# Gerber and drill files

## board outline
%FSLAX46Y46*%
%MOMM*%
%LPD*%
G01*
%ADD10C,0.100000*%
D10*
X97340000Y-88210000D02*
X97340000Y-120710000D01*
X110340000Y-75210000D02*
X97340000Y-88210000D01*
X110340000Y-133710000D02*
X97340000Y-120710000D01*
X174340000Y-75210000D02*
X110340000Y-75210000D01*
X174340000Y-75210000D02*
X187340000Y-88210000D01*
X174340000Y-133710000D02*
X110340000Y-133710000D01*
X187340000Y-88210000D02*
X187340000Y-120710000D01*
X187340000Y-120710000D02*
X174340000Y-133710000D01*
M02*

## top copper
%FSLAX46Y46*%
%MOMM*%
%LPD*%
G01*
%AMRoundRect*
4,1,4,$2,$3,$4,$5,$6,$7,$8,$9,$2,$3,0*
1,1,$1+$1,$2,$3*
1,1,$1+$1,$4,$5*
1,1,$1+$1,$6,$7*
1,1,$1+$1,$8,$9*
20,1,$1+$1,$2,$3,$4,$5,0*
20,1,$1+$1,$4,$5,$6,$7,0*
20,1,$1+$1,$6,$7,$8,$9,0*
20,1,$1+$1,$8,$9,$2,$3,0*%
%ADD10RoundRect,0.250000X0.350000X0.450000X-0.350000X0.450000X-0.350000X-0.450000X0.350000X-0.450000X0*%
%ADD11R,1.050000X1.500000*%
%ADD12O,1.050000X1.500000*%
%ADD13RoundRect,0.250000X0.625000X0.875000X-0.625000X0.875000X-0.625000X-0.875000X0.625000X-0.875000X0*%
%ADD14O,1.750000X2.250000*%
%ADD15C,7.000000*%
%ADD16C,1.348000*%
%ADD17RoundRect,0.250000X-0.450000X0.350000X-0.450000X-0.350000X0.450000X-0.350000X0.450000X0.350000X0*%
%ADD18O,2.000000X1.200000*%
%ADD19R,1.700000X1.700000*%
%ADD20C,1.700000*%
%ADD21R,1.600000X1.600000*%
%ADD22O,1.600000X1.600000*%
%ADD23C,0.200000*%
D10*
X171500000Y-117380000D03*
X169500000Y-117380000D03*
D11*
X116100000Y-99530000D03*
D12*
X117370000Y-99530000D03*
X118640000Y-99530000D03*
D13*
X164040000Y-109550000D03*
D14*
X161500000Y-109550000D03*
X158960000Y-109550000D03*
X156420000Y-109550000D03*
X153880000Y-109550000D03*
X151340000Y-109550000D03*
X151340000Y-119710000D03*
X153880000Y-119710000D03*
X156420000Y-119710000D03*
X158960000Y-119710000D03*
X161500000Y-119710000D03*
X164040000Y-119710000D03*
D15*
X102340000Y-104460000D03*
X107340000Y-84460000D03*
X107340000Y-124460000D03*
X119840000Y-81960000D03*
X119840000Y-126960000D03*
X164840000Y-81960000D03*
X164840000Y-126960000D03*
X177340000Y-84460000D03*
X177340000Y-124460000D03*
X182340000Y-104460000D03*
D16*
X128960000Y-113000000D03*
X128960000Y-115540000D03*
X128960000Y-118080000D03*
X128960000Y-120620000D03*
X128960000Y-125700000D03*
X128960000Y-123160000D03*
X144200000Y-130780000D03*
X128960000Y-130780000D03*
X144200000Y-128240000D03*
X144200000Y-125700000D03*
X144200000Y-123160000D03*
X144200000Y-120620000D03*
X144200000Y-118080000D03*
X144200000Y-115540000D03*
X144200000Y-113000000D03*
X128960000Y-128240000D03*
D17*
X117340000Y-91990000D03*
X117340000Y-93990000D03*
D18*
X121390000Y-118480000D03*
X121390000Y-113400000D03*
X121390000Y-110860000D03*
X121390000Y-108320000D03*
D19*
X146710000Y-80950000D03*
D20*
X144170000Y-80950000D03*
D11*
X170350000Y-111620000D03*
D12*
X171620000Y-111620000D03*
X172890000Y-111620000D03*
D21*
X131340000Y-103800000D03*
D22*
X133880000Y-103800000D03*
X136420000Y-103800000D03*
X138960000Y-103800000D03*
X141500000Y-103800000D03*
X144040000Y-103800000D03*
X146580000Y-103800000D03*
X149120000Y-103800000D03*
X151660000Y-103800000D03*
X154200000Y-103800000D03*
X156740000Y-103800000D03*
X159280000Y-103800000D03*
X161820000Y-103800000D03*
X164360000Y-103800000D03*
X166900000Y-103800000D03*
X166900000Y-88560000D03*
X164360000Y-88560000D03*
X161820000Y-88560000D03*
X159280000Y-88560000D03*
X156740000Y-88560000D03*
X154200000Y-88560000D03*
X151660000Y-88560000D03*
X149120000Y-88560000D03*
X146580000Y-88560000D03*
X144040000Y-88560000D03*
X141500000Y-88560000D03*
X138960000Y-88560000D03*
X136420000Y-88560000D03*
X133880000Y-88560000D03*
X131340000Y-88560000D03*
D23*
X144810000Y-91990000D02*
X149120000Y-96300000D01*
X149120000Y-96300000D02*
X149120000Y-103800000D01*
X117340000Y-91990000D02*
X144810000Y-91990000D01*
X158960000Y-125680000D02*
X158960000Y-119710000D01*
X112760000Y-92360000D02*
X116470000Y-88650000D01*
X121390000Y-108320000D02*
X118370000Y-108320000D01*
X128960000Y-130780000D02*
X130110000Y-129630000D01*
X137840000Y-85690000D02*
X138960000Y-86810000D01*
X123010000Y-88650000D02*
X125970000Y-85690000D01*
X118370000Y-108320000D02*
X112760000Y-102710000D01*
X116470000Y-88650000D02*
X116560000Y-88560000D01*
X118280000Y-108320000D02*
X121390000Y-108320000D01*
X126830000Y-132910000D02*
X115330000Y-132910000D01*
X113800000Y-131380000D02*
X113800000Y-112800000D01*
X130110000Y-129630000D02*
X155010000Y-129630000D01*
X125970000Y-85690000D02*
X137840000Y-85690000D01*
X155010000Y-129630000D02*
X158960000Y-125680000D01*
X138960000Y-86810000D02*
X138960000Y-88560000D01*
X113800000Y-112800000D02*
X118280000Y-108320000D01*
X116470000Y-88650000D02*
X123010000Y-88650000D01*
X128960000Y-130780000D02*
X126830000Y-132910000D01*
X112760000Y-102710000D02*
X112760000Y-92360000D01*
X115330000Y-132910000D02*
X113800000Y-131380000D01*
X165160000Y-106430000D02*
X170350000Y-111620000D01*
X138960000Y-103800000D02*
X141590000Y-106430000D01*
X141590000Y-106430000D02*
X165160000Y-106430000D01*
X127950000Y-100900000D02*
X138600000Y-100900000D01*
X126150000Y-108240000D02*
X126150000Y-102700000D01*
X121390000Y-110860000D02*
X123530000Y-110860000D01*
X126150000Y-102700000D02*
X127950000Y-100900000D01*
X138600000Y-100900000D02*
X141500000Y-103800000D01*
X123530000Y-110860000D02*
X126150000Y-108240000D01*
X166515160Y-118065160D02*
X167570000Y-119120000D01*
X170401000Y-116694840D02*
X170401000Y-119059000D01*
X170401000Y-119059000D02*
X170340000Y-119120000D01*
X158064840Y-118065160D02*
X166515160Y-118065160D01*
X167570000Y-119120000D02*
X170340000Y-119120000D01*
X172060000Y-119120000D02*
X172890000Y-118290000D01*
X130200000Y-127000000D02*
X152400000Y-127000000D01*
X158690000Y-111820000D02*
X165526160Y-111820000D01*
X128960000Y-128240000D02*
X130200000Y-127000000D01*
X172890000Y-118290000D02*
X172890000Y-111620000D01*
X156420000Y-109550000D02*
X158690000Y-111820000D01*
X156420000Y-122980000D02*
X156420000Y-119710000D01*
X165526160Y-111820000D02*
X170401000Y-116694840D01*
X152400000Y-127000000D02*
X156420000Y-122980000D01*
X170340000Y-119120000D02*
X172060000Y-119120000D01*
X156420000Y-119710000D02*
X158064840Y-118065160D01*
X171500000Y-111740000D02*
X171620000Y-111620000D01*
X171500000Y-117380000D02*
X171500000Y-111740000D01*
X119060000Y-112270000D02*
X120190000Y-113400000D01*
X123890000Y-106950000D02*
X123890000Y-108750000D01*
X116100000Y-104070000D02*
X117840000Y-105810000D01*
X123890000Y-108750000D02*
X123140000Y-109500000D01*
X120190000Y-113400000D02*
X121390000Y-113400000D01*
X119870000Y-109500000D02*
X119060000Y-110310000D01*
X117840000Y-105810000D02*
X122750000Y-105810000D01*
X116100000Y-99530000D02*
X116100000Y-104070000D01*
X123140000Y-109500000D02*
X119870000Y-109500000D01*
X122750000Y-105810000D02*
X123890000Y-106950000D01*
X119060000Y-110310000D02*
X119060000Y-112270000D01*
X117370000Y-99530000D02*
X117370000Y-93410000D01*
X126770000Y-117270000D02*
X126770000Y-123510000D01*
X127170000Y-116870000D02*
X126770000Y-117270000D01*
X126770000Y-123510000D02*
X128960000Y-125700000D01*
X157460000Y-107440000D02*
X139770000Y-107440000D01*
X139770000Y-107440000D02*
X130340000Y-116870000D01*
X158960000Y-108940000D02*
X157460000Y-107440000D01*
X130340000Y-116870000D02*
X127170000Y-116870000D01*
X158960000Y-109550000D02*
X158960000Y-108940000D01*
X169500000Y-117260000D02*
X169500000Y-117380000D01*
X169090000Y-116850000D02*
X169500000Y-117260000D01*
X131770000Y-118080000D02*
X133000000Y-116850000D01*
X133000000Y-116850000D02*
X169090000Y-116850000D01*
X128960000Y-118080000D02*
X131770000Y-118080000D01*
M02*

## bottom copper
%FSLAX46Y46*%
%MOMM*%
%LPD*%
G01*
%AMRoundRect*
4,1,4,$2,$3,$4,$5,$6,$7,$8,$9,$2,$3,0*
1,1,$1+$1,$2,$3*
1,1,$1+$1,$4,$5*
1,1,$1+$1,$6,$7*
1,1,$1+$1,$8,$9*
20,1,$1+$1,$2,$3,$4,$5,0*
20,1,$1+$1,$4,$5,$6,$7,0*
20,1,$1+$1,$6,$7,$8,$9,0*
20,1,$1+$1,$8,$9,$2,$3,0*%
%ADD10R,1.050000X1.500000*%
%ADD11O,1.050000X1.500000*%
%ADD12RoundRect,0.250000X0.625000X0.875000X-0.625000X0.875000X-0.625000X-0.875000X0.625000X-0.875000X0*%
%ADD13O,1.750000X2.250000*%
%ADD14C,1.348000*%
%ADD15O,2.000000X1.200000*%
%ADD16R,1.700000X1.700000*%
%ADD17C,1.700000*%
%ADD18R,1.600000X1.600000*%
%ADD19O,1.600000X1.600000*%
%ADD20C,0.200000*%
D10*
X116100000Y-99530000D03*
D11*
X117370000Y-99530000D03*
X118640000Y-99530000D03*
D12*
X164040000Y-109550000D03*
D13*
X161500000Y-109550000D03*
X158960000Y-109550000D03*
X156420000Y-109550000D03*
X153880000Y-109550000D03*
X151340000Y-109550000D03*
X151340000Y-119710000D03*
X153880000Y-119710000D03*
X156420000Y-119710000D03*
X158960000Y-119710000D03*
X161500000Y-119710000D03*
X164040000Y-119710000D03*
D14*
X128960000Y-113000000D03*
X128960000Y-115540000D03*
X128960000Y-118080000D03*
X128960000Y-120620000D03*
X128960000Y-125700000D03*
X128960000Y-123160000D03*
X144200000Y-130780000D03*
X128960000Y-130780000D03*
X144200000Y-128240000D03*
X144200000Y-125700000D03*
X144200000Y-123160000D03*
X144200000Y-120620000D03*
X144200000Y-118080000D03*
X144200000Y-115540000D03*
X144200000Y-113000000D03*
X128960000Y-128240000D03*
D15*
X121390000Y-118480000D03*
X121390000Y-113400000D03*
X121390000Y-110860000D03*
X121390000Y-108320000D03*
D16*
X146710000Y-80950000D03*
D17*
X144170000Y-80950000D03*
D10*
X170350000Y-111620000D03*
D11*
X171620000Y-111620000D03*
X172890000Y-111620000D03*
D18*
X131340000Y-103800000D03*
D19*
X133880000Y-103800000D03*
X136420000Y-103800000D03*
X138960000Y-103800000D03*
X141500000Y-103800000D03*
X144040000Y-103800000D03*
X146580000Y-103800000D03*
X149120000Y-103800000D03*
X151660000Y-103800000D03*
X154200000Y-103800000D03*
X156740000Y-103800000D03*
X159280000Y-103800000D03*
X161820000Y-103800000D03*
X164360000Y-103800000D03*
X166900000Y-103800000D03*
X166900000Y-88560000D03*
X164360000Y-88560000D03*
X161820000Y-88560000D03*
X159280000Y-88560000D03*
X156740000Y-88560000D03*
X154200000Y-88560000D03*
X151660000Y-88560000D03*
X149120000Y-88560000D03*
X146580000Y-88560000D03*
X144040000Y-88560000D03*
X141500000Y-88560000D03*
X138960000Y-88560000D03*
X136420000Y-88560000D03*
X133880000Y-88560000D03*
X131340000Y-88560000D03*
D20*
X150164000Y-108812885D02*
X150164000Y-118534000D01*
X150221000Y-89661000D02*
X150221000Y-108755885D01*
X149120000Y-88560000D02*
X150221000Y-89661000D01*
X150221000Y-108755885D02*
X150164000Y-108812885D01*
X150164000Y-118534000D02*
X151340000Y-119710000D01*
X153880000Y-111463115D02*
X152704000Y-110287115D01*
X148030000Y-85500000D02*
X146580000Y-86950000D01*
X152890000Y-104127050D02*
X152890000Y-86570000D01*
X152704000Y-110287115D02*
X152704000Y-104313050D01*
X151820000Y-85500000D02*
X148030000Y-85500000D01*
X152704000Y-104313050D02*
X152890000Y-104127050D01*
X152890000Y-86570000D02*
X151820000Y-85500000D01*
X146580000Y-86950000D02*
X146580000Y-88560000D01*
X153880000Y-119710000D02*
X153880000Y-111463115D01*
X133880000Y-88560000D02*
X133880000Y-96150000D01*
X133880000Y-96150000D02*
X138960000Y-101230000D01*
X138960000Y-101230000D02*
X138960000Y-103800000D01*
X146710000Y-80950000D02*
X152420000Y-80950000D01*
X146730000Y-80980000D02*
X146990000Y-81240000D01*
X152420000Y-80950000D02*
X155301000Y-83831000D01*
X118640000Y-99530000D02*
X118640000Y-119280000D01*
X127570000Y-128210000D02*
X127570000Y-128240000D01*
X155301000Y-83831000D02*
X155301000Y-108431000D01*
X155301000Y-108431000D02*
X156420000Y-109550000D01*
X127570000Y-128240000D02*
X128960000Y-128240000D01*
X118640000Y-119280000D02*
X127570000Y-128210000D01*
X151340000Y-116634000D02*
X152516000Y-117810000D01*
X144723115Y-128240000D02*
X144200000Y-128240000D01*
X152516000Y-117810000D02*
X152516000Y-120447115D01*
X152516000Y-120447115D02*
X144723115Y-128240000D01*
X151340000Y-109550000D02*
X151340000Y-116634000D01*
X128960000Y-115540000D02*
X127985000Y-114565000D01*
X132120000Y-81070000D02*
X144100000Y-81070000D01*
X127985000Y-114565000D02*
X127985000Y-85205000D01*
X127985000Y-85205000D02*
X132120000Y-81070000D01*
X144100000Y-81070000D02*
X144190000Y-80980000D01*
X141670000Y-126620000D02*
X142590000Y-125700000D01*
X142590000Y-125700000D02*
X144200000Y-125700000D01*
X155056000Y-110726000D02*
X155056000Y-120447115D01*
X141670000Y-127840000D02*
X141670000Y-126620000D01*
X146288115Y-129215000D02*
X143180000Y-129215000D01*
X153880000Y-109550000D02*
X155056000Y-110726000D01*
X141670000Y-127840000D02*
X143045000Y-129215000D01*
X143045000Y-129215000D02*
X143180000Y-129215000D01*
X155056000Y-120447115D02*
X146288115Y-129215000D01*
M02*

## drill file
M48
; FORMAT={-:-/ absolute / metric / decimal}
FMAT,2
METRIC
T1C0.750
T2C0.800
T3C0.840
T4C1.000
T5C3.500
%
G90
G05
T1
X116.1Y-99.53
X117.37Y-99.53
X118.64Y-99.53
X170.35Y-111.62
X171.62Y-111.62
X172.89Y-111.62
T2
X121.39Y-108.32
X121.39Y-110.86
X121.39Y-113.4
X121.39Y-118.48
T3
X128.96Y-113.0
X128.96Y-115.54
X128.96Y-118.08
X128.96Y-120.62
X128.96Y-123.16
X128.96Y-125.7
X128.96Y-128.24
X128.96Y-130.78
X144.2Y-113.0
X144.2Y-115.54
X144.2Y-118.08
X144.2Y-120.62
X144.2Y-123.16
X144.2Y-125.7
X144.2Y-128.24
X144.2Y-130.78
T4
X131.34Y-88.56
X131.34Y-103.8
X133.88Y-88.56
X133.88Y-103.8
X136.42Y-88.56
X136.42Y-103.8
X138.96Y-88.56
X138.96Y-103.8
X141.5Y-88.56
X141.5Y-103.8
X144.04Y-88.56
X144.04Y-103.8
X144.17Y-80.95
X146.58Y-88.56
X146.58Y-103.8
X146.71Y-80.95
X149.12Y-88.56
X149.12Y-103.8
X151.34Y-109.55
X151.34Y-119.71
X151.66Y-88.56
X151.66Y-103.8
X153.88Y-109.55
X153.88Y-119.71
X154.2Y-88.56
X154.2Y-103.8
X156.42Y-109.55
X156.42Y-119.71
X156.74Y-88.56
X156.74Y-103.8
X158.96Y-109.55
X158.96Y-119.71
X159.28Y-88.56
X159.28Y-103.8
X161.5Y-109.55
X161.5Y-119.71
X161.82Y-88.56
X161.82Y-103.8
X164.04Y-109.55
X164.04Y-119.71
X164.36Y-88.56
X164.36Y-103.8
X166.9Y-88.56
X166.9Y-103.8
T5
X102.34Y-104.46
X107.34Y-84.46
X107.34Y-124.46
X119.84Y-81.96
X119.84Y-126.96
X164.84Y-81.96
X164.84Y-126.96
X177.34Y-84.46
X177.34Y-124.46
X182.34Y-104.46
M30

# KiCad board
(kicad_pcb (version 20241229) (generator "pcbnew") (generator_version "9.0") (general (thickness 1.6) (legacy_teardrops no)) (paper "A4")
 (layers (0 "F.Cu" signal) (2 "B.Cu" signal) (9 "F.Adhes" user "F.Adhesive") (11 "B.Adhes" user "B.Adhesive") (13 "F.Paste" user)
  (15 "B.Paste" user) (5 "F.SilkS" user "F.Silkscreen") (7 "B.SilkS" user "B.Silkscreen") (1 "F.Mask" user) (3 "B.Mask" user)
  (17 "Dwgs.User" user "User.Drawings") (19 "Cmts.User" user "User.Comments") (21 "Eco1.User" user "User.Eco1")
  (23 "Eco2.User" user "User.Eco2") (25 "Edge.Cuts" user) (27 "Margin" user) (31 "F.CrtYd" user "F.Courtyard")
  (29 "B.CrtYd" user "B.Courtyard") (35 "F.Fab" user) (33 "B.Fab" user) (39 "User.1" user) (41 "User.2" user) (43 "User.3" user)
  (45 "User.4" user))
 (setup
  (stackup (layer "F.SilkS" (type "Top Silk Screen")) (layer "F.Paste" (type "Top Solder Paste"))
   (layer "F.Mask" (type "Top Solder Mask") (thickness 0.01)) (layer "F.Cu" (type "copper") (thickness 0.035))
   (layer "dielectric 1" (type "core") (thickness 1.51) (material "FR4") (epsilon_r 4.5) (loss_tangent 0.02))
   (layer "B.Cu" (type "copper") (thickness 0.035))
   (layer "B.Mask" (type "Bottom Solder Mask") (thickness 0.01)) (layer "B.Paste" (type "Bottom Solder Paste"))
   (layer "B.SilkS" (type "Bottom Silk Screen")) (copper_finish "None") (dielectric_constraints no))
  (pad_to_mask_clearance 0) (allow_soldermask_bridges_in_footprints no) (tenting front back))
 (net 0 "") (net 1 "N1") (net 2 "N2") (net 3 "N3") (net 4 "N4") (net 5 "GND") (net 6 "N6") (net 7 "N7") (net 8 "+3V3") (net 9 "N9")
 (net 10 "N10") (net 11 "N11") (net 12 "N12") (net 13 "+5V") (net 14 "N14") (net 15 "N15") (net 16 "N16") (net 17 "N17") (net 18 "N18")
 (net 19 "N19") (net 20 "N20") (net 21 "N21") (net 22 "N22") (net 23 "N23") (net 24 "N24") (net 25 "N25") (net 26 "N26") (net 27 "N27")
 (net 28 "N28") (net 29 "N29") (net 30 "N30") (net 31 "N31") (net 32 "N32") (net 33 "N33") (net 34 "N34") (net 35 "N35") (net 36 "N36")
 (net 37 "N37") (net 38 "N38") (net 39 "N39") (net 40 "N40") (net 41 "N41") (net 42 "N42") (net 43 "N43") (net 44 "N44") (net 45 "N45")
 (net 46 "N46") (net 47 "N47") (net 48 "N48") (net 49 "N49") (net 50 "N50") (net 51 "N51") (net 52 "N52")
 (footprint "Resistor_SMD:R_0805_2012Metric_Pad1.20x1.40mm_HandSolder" (layer "F.Cu") (at 170.5 117.38 180)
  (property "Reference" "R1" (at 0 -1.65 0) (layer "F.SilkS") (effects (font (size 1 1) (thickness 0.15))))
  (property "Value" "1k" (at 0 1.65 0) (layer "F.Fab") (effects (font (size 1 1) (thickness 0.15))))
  (pad "1" smd roundrect (at -1 0 180) (size 1.2 1.4) (layers "F.Cu" "F.Mask" "F.Paste") (roundrect_rratio 0.208333) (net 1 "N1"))
  (pad "2" smd roundrect (at 1 0 180) (size 1.2 1.4) (layers "F.Cu" "F.Mask" "F.Paste") (roundrect_rratio 0.208333) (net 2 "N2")))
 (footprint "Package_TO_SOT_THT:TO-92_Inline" (layer "F.Cu") (at 116.1 99.53)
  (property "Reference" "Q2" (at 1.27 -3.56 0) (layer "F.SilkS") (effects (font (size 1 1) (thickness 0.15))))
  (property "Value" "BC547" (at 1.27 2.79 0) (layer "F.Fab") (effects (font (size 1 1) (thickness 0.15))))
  (pad "1" thru_hole rect (at 0 0) (size 1.05 1.5) (drill 0.75) (layers "*.Cu" "*.Mask") (remove_unused_layers no) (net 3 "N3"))
  (pad "2" thru_hole oval (at 1.27 0) (size 1.05 1.5) (drill 0.75) (layers "*.Cu" "*.Mask") (remove_unused_layers no) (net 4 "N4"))
  (pad "3" thru_hole oval (at 2.54 0) (size 1.05 1.5) (drill 0.75) (layers "*.Cu" "*.Mask") (remove_unused_layers no) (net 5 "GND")))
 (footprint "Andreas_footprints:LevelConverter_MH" (layer "F.Cu") (at 157.69 114.63 180)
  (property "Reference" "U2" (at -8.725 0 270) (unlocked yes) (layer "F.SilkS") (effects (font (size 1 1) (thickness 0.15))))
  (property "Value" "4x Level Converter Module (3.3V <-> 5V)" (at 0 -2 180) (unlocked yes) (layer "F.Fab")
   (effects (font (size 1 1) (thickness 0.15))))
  (pad "1" thru_hole roundrect (at -6.35 5.08 180) (size 1.75 2.25) (drill 1) (layers "*.Cu" "*.Mask") (remove_unused_layers no)
   (roundrect_rratio 0.1428571429) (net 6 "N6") (thermal_bridge_angle 45))
  (pad "2" thru_hole oval (at -3.81 5.08 180) (size 1.75 2.25) (drill 1) (layers "*.Cu" "*.Mask") (remove_unused_layers no) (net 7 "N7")
   (thermal_bridge_angle 45))
  (pad "3" thru_hole oval (at -1.27 5.08 180) (size 1.75 2.25) (drill 1) (layers "*.Cu" "*.Mask") (remove_unused_layers no) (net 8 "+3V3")
   (thermal_bridge_angle 45))
  (pad "4" thru_hole oval (at 1.27 5.08 180) (size 1.75 2.25) (drill 1) (layers "*.Cu" "*.Mask") (remove_unused_layers no) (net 5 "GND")
   (thermal_bridge_angle 45))
  (pad "5" thru_hole oval (at 3.81 5.08 180) (size 1.75 2.25) (drill 1) (layers "*.Cu" "*.Mask") (remove_unused_layers no) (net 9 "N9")
   (thermal_bridge_angle 45))
  (pad "6" thru_hole oval (at 6.35 5.08 180) (size 1.75 2.25) (drill 1) (layers "*.Cu" "*.Mask") (remove_unused_layers no) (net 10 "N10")
   (thermal_bridge_angle 45))
  (pad "7" thru_hole oval (at 6.35 -5.08 180) (size 1.75 2.25) (drill 1) (layers "*.Cu" "*.Mask") (remove_unused_layers no) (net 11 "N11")
   (thermal_bridge_angle 45))
  (pad "8" thru_hole oval (at 3.81 -5.08 180) (size 1.75 2.25) (drill 1) (layers "*.Cu" "*.Mask") (remove_unused_layers no) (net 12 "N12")
   (thermal_bridge_angle 45))
  (pad "9" thru_hole oval (at 1.27 -5.08 180) (size 1.75 2.25) (drill 1) (layers "*.Cu" "*.Mask") (remove_unused_layers no) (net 5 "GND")
   (thermal_bridge_angle 45))
  (pad "10" thru_hole oval (at -1.27 -5.08 180) (size 1.75 2.25) (drill 1) (layers "*.Cu" "*.Mask") (remove_unused_layers no) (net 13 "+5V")
   (thermal_bridge_angle 45))
  (pad "11" thru_hole oval (at -3.81 -5.08 180) (size 1.75 2.25) (drill 1) (layers "*.Cu" "*.Mask") (remove_unused_layers no) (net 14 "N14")
   (thermal_bridge_angle 45))
  (pad "12" thru_hole oval (at -6.35 -5.08 180) (size 1.75 2.25) (drill 1) (layers "*.Cu" "*.Mask") (remove_unused_layers no) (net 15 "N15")
   (thermal_bridge_angle 45)))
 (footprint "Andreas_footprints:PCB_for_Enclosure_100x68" (layer "F.Cu") (at 142.34 104.46)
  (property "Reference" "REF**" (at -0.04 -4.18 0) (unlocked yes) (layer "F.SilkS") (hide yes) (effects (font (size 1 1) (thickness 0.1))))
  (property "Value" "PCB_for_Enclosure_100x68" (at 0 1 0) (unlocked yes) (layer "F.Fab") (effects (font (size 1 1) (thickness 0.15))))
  (fp_line (start -45 -16.25) (end -45 16.25) (stroke (width 0.1) (type default)) (layer "Edge.Cuts"))
  (fp_line (start -32 -29.25) (end -45 -16.25) (stroke (width 0.1) (type default)) (layer "Edge.Cuts"))
  (fp_line (start -32 29.25) (end -45 16.25) (stroke (width 0.1) (type default)) (layer "Edge.Cuts"))
  (fp_line (start 32 -29.25) (end -32 -29.25) (stroke (width 0.1) (type default)) (layer "Edge.Cuts"))
  (fp_line (start 32 -29.25) (end 45 -16.25) (stroke (width 0.1) (type default)) (layer "Edge.Cuts"))
  (fp_line (start 32 29.25) (end -32 29.25) (stroke (width 0.1) (type default)) (layer "Edge.Cuts"))
  (fp_line (start 45 -16.25) (end 45 16.25) (stroke (width 0.1) (type default)) (layer "Edge.Cuts"))
  (fp_line (start 45 16.25) (end 32 29.25) (stroke (width 0.1) (type default)) (layer "Edge.Cuts"))
  (pad "" np_thru_hole circle (at -40 0) (size 7 7) (drill 3.5) (layers "F.Cu" "F.Mask" "F.Paste"))
  (pad "" np_thru_hole circle (at -35 -20) (size 7 7) (drill 3.5) (layers "F.Cu" "F.Mask" "F.Paste"))
  (pad "" np_thru_hole circle (at -35 20) (size 7 7) (drill 3.5) (layers "F.Cu" "F.Mask" "F.Paste"))
  (pad "" np_thru_hole circle (at -22.5 -22.5) (size 7 7) (drill 3.5) (layers "F.Cu" "F.Mask" "F.Paste"))
  (pad "" np_thru_hole circle (at -22.5 22.5) (size 7 7) (drill 3.5) (layers "F.Cu" "F.Mask" "F.Paste"))
  (pad "" np_thru_hole circle (at 22.5 -22.5) (size 7 7) (drill 3.5) (layers "F.Cu" "F.Mask" "F.Paste"))
  (pad "" np_thru_hole circle (at 22.5 22.5) (size 7 7) (drill 3.5) (layers "F.Cu" "F.Mask" "F.Paste"))
  (pad "" np_thru_hole circle (at 35 -20) (size 7 7) (drill 3.5) (layers "F.Cu" "F.Mask" "F.Paste"))
  (pad "" np_thru_hole circle (at 35 20) (size 7 7) (drill 3.5) (layers "F.Cu" "F.Mask" "F.Paste"))
  (pad "" np_thru_hole circle (at 40 0) (size 7 7) (drill 3.5) (layers "F.Cu" "F.Mask" "F.Paste")))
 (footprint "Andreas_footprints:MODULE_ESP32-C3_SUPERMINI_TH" (layer "F.Cu") (at 136.58 120.88 180)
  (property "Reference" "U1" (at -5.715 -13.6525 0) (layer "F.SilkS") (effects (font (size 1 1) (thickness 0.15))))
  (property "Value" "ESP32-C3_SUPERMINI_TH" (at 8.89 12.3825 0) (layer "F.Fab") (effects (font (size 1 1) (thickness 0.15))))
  (pad "0" thru_hole circle (at 7.62 7.88 180) (size 1.348 1.348) (drill 0.84) (layers "*.Cu" "*.Mask") (remove_unused_layers no)
   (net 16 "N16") (solder_mask_margin 0.102))
  (pad "1" thru_hole circle (at 7.62 5.34 180) (size 1.348 1.348) (drill 0.84) (layers "*.Cu" "*.Mask") (remove_unused_layers no)
   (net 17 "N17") (solder_mask_margin 0.102))
  (pad "2" thru_hole circle (at 7.62 2.8 180) (size 1.348 1.348) (drill 0.84) (layers "*.Cu" "*.Mask") (remove_unused_layers no)
   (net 2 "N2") (solder_mask_margin 0.102))
  (pad "3" thru_hole circle (at 7.62 0.26 180) (size 1.348 1.348) (drill 0.84) (layers "*.Cu" "*.Mask") (remove_unused_layers no)
   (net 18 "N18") (solder_mask_margin 0.102))
  (pad "3.3" thru_hole circle (at 7.62 -4.82 180) (size 1.348 1.348) (drill 0.84) (layers "*.Cu" "*.Mask") (remove_unused_layers no)
   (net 8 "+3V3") (solder_mask_margin 0.102))
  (pad "4" thru_hole circle (at 7.62 -2.28 180) (size 1.348 1.348) (drill 0.84) (layers "*.Cu" "*.Mask") (remove_unused_layers no)
   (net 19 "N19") (solder_mask_margin 0.102))
  (pad "5" thru_hole circle (at -7.62 -9.9 180) (size 1.348 1.348) (drill 0.84) (layers "*.Cu" "*.Mask") (remove_unused_layers no)
   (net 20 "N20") (solder_mask_margin 0.102))
  (pad "5V" thru_hole circle (at 7.62 -9.9 180) (size 1.348 1.348) (drill 0.84) (layers "*.Cu" "*.Mask") (remove_unused_layers no)
   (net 13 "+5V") (solder_mask_margin 0.102))
  (pad "6" thru_hole circle (at -7.62 -7.36 180) (size 1.348 1.348) (drill 0.84) (layers "*.Cu" "*.Mask") (remove_unused_layers no)
   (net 10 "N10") (solder_mask_margin 0.102))
  (pad "7" thru_hole circle (at -7.62 -4.82 180) (size 1.348 1.348) (drill 0.84) (layers "*.Cu" "*.Mask") (remove_unused_layers no)
   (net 9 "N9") (solder_mask_margin 0.102))
  (pad "8" thru_hole circle (at -7.62 -2.28 180) (size 1.348 1.348) (drill 0.84) (layers "*.Cu" "*.Mask") (remove_unused_layers no)
   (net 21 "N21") (solder_mask_margin 0.102))
  (pad "9" thru_hole circle (at -7.62 0.26 180) (size 1.348 1.348) (drill 0.84) (layers "*.Cu" "*.Mask") (remove_unused_layers no)
   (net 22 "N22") (solder_mask_margin 0.102))
  (pad "10" thru_hole circle (at -7.62 2.8 180) (size 1.348 1.348) (drill 0.84) (layers "*.Cu" "*.Mask") (remove_unused_layers no)
   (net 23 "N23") (solder_mask_margin 0.102))
  (pad "20" thru_hole circle (at -7.62 5.34 180) (size 1.348 1.348) (drill 0.84) (layers "*.Cu" "*.Mask") (remove_unused_layers no)
   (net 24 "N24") (solder_mask_margin 0.102))
  (pad "21" thru_hole circle (at -7.62 7.88 180) (size 1.348 1.348) (drill 0.84) (layers "*.Cu" "*.Mask") (remove_unused_layers no)
   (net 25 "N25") (solder_mask_margin 0.102))
  (pad "G" thru_hole circle (at 7.62 -7.36 180) (size 1.348 1.348) (drill 0.84) (layers "*.Cu" "*.Mask") (remove_unused_layers no)
   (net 5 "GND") (solder_mask_margin 0.102)))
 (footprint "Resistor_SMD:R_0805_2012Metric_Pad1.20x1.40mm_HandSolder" (layer "F.Cu") (at 117.34 92.99 -90)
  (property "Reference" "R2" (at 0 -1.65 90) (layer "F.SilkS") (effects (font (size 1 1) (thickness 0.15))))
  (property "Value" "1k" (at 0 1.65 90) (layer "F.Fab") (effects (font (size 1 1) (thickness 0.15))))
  (pad "1" smd roundrect (at -1 0 270) (size 1.2 1.4) (layers "F.Cu" "F.Mask" "F.Paste") (roundrect_rratio 0.208333) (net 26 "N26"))
  (pad "2" smd roundrect (at 1 0 270) (size 1.2 1.4) (layers "F.Cu" "F.Mask" "F.Paste") (roundrect_rratio 0.208333) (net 4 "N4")))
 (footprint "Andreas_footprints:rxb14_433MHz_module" (layer "F.Cu") (at 121.39 113.4 90)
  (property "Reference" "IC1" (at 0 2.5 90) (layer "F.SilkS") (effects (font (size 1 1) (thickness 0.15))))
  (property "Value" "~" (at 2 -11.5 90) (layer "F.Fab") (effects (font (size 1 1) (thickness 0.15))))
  (pad "1" thru_hole oval (at -5.08 0 90) (size 1.2 2) (drill 0.8) (layers "*.Cu" "*.Mask") (remove_unused_layers no) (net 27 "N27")
   (thermal_bridge_angle 45))
  (pad "2" thru_hole oval (at 0 0 90) (size 1.2 2) (drill 0.8) (layers "*.Cu" "*.Mask") (remove_unused_layers no) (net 3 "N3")
   (thermal_bridge_angle 45))
  (pad "3" thru_hole oval (at 2.54 0 90) (size 1.2 2) (drill 0.8) (layers "*.Cu" "*.Mask") (remove_unused_layers no) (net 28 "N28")
   (thermal_bridge_angle 45))
  (pad "4" thru_hole oval (at 5.08 0 90) (size 1.2 2) (drill 0.8) (layers "*.Cu" "*.Mask") (remove_unused_layers no) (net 13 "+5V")
   (thermal_bridge_angle 45)))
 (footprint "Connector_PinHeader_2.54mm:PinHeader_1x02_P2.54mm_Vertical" (layer "F.Cu") (at 146.71 80.95 -90)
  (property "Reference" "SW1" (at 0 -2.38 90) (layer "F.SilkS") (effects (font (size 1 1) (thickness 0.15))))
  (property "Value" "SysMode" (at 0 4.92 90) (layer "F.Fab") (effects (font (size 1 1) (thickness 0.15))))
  (pad "1" thru_hole rect (at 0 0 270) (size 1.7 1.7) (drill 1) (layers "*.Cu" "*.Mask") (remove_unused_layers no) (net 5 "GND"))
  (pad "2" thru_hole circle (at 0 2.54 270) (size 1.7 1.7) (drill 1) (layers "*.Cu" "*.Mask") (remove_unused_layers no) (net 17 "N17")))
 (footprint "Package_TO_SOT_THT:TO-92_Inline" (layer "F.Cu") (at 170.35 111.62)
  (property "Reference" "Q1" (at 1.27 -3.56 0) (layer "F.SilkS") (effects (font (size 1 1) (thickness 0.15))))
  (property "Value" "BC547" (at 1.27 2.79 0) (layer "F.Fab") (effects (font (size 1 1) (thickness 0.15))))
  (pad "1" thru_hole rect (at 0 0) (size 1.05 1.5) (drill 0.75) (layers "*.Cu" "*.Mask") (remove_unused_layers no) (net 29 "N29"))
  (pad "2" thru_hole oval (at 1.27 0) (size 1.05 1.5) (drill 0.75) (layers "*.Cu" "*.Mask") (remove_unused_layers no) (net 1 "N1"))
  (pad "3" thru_hole oval (at 2.54 0) (size 1.05 1.5) (drill 0.75) (layers "*.Cu" "*.Mask") (remove_unused_layers no) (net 5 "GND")))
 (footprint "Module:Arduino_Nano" (layer "F.Cu") (at 131.34 103.8 90)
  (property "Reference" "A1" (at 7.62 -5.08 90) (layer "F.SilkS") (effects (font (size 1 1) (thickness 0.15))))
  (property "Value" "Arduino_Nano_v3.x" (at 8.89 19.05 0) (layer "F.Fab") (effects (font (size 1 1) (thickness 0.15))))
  (pad "1" thru_hole rect (at 0 0 90) (size 1.6 1.6) (drill 1) (layers "*.Cu" "*.Mask") (remove_unused_layers no) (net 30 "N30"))
  (pad "2" thru_hole oval (at 0 2.54 90) (size 1.6 1.6) (drill 1) (layers "*.Cu" "*.Mask") (remove_unused_layers no) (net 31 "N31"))
  (pad "3" thru_hole oval (at 0 5.08 90) (size 1.6 1.6) (drill 1) (layers "*.Cu" "*.Mask") (remove_unused_layers no) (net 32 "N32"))
  (pad "4" thru_hole oval (at 0 7.62 90) (size 1.6 1.6) (drill 1) (layers "*.Cu" "*.Mask") (remove_unused_layers no) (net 29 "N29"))
  (pad "5" thru_hole oval (at 0 10.16 90) (size 1.6 1.6) (drill 1) (layers "*.Cu" "*.Mask") (remove_unused_layers no) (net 28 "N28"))
  (pad "6" thru_hole oval (at 0 12.7 90) (size 1.6 1.6) (drill 1) (layers "*.Cu" "*.Mask") (remove_unused_layers no) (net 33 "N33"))
  (pad "7" thru_hole oval (at 0 15.24 90) (size 1.6 1.6) (drill 1) (layers "*.Cu" "*.Mask") (remove_unused_layers no) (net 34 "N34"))
  (pad "8" thru_hole oval (at 0 17.78 90) (size 1.6 1.6) (drill 1) (layers "*.Cu" "*.Mask") (remove_unused_layers no) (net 26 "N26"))
  (pad "9" thru_hole oval (at 0 20.32 90) (size 1.6 1.6) (drill 1) (layers "*.Cu" "*.Mask") (remove_unused_layers no) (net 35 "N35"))
  (pad "10" thru_hole oval (at 0 22.86 90) (size 1.6 1.6) (drill 1) (layers "*.Cu" "*.Mask") (remove_unused_layers no) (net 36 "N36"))
  (pad "11" thru_hole oval (at 0 25.4 90) (size 1.6 1.6) (drill 1) (layers "*.Cu" "*.Mask") (remove_unused_layers no) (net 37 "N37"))
  (pad "12" thru_hole oval (at 0 27.94 90) (size 1.6 1.6) (drill 1) (layers "*.Cu" "*.Mask") (remove_unused_layers no) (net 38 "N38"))
  (pad "13" thru_hole oval (at 0 30.48 90) (size 1.6 1.6) (drill 1) (layers "*.Cu" "*.Mask") (remove_unused_layers no) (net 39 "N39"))
  (pad "14" thru_hole oval (at 0 33.02 90) (size 1.6 1.6) (drill 1) (layers "*.Cu" "*.Mask") (remove_unused_layers no) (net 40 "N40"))
  (pad "15" thru_hole oval (at 0 35.56 90) (size 1.6 1.6) (drill 1) (layers "*.Cu" "*.Mask") (remove_unused_layers no) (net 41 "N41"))
  (pad "16" thru_hole oval (at 15.24 35.56 90) (size 1.6 1.6) (drill 1) (layers "*.Cu" "*.Mask") (remove_unused_layers no) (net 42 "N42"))
  (pad "17" thru_hole oval (at 15.24 33.02 90) (size 1.6 1.6) (drill 1) (layers "*.Cu" "*.Mask") (remove_unused_layers no) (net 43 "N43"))
  (pad "18" thru_hole oval (at 15.24 30.48 90) (size 1.6 1.6) (drill 1) (layers "*.Cu" "*.Mask") (remove_unused_layers no) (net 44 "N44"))
  (pad "19" thru_hole oval (at 15.24 27.94 90) (size 1.6 1.6) (drill 1) (layers "*.Cu" "*.Mask") (remove_unused_layers no) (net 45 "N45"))
  (pad "20" thru_hole oval (at 15.24 25.4 90) (size 1.6 1.6) (drill 1) (layers "*.Cu" "*.Mask") (remove_unused_layers no) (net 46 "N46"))
  (pad "21" thru_hole oval (at 15.24 22.86 90) (size 1.6 1.6) (drill 1) (layers "*.Cu" "*.Mask") (remove_unused_layers no) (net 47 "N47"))
  (pad "22" thru_hole oval (at 15.24 20.32 90) (size 1.6 1.6) (drill 1) (layers "*.Cu" "*.Mask") (remove_unused_layers no) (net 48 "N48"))
  (pad "23" thru_hole oval (at 15.24 17.78 90) (size 1.6 1.6) (drill 1) (layers "*.Cu" "*.Mask") (remove_unused_layers no) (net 11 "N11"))
  (pad "24" thru_hole oval (at 15.24 15.24 90) (size 1.6 1.6) (drill 1) (layers "*.Cu" "*.Mask") (remove_unused_layers no) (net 12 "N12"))
  (pad "25" thru_hole oval (at 15.24 12.7 90) (size 1.6 1.6) (drill 1) (layers "*.Cu" "*.Mask") (remove_unused_layers no) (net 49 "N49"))
  (pad "26" thru_hole oval (at 15.24 10.16 90) (size 1.6 1.6) (drill 1) (layers "*.Cu" "*.Mask") (remove_unused_layers no) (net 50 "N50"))
  (pad "27" thru_hole oval (at 15.24 7.62 90) (size 1.6 1.6) (drill 1) (layers "*.Cu" "*.Mask") (remove_unused_layers no) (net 13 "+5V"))
  (pad "28" thru_hole oval (at 15.24 5.08 90) (size 1.6 1.6) (drill 1) (layers "*.Cu" "*.Mask") (remove_unused_layers no) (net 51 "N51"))
  (pad "29" thru_hole oval (at 15.24 2.54 90) (size 1.6 1.6) (drill 1) (layers "*.Cu" "*.Mask") (remove_unused_layers no) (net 29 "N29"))
  (pad "30" thru_hole oval (at 15.24 0 90) (size 1.6 1.6) (drill 1) (layers "*.Cu" "*.Mask") (remove_unused_layers no) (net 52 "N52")))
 (segment (start 144.81 91.99) (end 149.12 96.3) (width 0.2) (layer "F.Cu") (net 26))
 (segment (start 149.12 96.3) (end 149.12 103.8) (width 0.2) (layer "F.Cu") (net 26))
 (segment (start 117.34 91.99) (end 144.81 91.99) (width 0.2) (layer "F.Cu") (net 26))
 (segment (start 150.164 108.812885) (end 150.164 118.534) (width 0.2) (layer "B.Cu") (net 11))
 (segment (start 150.221 89.661) (end 150.221 108.755885) (width 0.2) (layer "B.Cu") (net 11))
 (segment (start 149.12 88.56) (end 150.221 89.661) (width 0.2) (layer "B.Cu") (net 11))
 (segment (start 150.221 108.755885) (end 150.164 108.812885) (width 0.2) (layer "B.Cu") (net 11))
 (segment (start 150.164 118.534) (end 151.34 119.71) (width 0.2) (layer "B.Cu") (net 11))
 (segment (start 153.88 111.463115) (end 152.704 110.287115) (width 0.2) (layer "B.Cu") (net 12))
 (segment (start 148.03 85.5) (end 146.58 86.95) (width 0.2) (layer "B.Cu") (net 12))
 (segment (start 152.89 104.12705) (end 152.89 86.57) (width 0.2) (layer "B.Cu") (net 12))
 (segment (start 152.704 110.287115) (end 152.704 104.31305) (width 0.2) (layer "B.Cu") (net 12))
 (segment (start 151.82 85.5) (end 148.03 85.5) (width 0.2) (layer "B.Cu") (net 12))
 (segment (start 152.704 104.31305) (end 152.89 104.12705) (width 0.2) (layer "B.Cu") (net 12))
 (segment (start 152.89 86.57) (end 151.82 85.5) (width 0.2) (layer "B.Cu") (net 12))
 (segment (start 146.58 86.95) (end 146.58 88.56) (width 0.2) (layer "B.Cu") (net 12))
 (segment (start 153.88 119.71) (end 153.88 111.463115) (width 0.2) (layer "B.Cu") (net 12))
 (segment (start 158.96 125.68) (end 158.96 119.71) (width 0.2) (layer "F.Cu") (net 13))
 (segment (start 112.76 92.36) (end 116.47 88.65) (width 0.2) (layer "F.Cu") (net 13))
 (segment (start 121.39 108.32) (end 118.37 108.32) (width 0.2) (layer "F.Cu") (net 13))
 (segment (start 128.96 130.78) (end 130.11 129.63) (width 0.2) (layer "F.Cu") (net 13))
 (segment (start 137.84 85.69) (end 138.96 86.81) (width 0.2) (layer "F.Cu") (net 13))
 (segment (start 123.01 88.65) (end 125.97 85.69) (width 0.2) (layer "F.Cu") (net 13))
 (segment (start 118.37 108.32) (end 112.76 102.71) (width 0.2) (layer "F.Cu") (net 13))
 (segment (start 116.47 88.65) (end 116.56 88.56) (width 0.2) (layer "F.Cu") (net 13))
 (segment (start 118.28 108.32) (end 121.39 108.32) (width 0.2) (layer "F.Cu") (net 13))
 (segment (start 126.83 132.91) (end 115.33 132.91) (width 0.2) (layer "F.Cu") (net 13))
 (segment (start 113.8 131.38) (end 113.8 112.8) (width 0.2) (layer "F.Cu") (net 13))
 (segment (start 130.11 129.63) (end 155.01 129.63) (width 0.2) (layer "F.Cu") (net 13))
 (segment (start 125.97 85.69) (end 137.84 85.69) (width 0.2) (layer "F.Cu") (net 13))
 (segment (start 155.01 129.63) (end 158.96 125.68) (width 0.2) (layer "F.Cu") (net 13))
 (segment (start 138.96 86.81) (end 138.96 88.56) (width 0.2) (layer "F.Cu") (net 13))
 (segment (start 113.8 112.8) (end 118.28 108.32) (width 0.2) (layer "F.Cu") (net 13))
 (segment (start 116.47 88.65) (end 123.01 88.65) (width 0.2) (layer "F.Cu") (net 13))
 (segment (start 128.96 130.78) (end 126.83 132.91) (width 0.2) (layer "F.Cu") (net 13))
 (segment (start 112.76 102.71) (end 112.76 92.36) (width 0.2) (layer "F.Cu") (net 13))
 (segment (start 115.33 132.91) (end 113.8 131.38) (width 0.2) (layer "F.Cu") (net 13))
 (segment (start 165.16 106.43) (end 170.35 111.62) (width 0.2) (layer "F.Cu") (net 29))
 (segment (start 138.96 103.8) (end 141.59 106.43) (width 0.2) (layer "F.Cu") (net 29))
 (segment (start 141.59 106.43) (end 165.16 106.43) (width 0.2) (layer "F.Cu") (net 29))
 (segment (start 133.88 88.56) (end 133.88 96.15) (width 0.2) (layer "B.Cu") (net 29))
 (segment (start 133.88 96.15) (end 138.96 101.23) (width 0.2) (layer "B.Cu") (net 29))
 (segment (start 138.96 101.23) (end 138.96 103.8) (width 0.2) (layer "B.Cu") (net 29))
 (segment (start 127.95 100.9) (end 138.6 100.9) (width 0.2) (layer "F.Cu") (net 28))
 (segment (start 126.15 108.24) (end 126.15 102.7) (width 0.2) (layer "F.Cu") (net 28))
 (segment (start 121.39 110.86) (end 123.53 110.86) (width 0.2) (layer "F.Cu") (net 28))
 (segment (start 126.15 102.7) (end 127.95 100.9) (width 0.2) (layer "F.Cu") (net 28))
 (segment (start 138.6 100.9) (end 141.5 103.8) (width 0.2) (layer "F.Cu") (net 28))
 (segment (start 123.53 110.86) (end 126.15 108.24) (width 0.2) (layer "F.Cu") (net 28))
 (segment (start 166.51516 118.06516) (end 167.57 119.12) (width 0.2) (layer "F.Cu") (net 5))
 (segment (start 170.401 116.69484) (end 170.401 119.059) (width 0.2) (layer "F.Cu") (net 5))
 (segment (start 170.401 119.059) (end 170.34 119.12) (width 0.2) (layer "F.Cu") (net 5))
 (segment (start 158.06484 118.06516) (end 166.51516 118.06516) (width 0.2) (layer "F.Cu") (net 5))
 (segment (start 167.57 119.12) (end 170.34 119.12) (width 0.2) (layer "F.Cu") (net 5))
 (segment (start 172.06 119.12) (end 172.89 118.29) (width 0.2) (layer "F.Cu") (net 5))
 (segment (start 130.2 127) (end 152.4 127) (width 0.2) (layer "F.Cu") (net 5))
 (segment (start 158.69 111.82) (end 165.52616 111.82) (width 0.2) (layer "F.Cu") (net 5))
 (segment (start 128.96 128.24) (end 130.2 127) (width 0.2) (layer "F.Cu") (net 5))
 (segment (start 172.89 118.29) (end 172.89 111.62) (width 0.2) (layer "F.Cu") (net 5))
 (segment (start 156.42 109.55) (end 158.69 111.82) (width 0.2) (layer "F.Cu") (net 5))
 (segment (start 156.42 122.98) (end 156.42 119.71) (width 0.2) (layer "F.Cu") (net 5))
 (segment (start 165.52616 111.82) (end 170.401 116.69484) (width 0.2) (layer "F.Cu") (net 5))
 (segment (start 152.4 127) (end 156.42 122.98) (width 0.2) (layer "F.Cu") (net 5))
 (segment (start 170.34 119.12) (end 172.06 119.12) (width 0.2) (layer "F.Cu") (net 5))
 (segment (start 156.42 119.71) (end 158.06484 118.06516) (width 0.2) (layer "F.Cu") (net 5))
 (segment (start 146.71 80.95) (end 152.42 80.95) (width 0.2) (layer "B.Cu") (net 5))
 (segment (start 146.73 80.98) (end 146.99 81.24) (width 0.2) (layer "B.Cu") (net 5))
 (segment (start 152.42 80.95) (end 155.301 83.831) (width 0.2) (layer "B.Cu") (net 5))
 (segment (start 118.64 99.53) (end 118.64 119.28) (width 0.2) (layer "B.Cu") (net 5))
 (segment (start 127.57 128.21) (end 127.57 128.24) (width 0.2) (layer "B.Cu") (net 5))
 (segment (start 155.301 83.831) (end 155.301 108.431) (width 0.2) (layer "B.Cu") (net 5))
 (segment (start 155.301 108.431) (end 156.42 109.55) (width 0.2) (layer "B.Cu") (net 5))
 (segment (start 127.57 128.24) (end 128.96 128.24) (width 0.2) (layer "B.Cu") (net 5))
 (segment (start 118.64 119.28) (end 127.57 128.21) (width 0.2) (layer "B.Cu") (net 5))
 (segment (start 171.5 111.74) (end 171.62 111.62) (width 0.2) (layer "F.Cu") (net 1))
 (segment (start 171.5 117.38) (end 171.5 111.74) (width 0.2) (layer "F.Cu") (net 1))
 (segment (start 119.06 112.27) (end 120.19 113.4) (width 0.2) (layer "F.Cu") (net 3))
 (segment (start 123.89 106.95) (end 123.89 108.75) (width 0.2) (layer "F.Cu") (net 3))
 (segment (start 116.1 104.07) (end 117.84 105.81) (width 0.2) (layer "F.Cu") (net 3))
 (segment (start 123.89 108.75) (end 123.14 109.5) (width 0.2) (layer "F.Cu") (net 3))
 (segment (start 120.19 113.4) (end 121.39 113.4) (width 0.2) (layer "F.Cu") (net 3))
 (segment (start 119.87 109.5) (end 119.06 110.31) (width 0.2) (layer "F.Cu") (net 3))
 (segment (start 117.84 105.81) (end 122.75 105.81) (width 0.2) (layer "F.Cu") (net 3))
 (segment (start 116.1 99.53) (end 116.1 104.07) (width 0.2) (layer "F.Cu") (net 3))
 (segment (start 123.14 109.5) (end 119.87 109.5) (width 0.2) (layer "F.Cu") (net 3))
 (segment (start 122.75 105.81) (end 123.89 106.95) (width 0.2) (layer "F.Cu") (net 3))
 (segment (start 119.06 110.31) (end 119.06 112.27) (width 0.2) (layer "F.Cu") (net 3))
 (segment (start 117.37 99.53) (end 117.37 93.41) (width 0.2) (layer "F.Cu") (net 4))
 (segment (start 126.77 117.27) (end 126.77 123.51) (width 0.2) (layer "F.Cu") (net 8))
 (segment (start 127.17 116.87) (end 126.77 117.27) (width 0.2) (layer "F.Cu") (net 8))
 (segment (start 126.77 123.51) (end 128.96 125.7) (width 0.2) (layer "F.Cu") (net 8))
 (segment (start 157.46 107.44) (end 139.77 107.44) (width 0.2) (layer "F.Cu") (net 8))
 (segment (start 139.77 107.44) (end 130.34 116.87) (width 0.2) (layer "F.Cu") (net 8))
 (segment (start 158.96 108.94) (end 157.46 107.44) (width 0.2) (layer "F.Cu") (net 8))
 (segment (start 130.34 116.87) (end 127.17 116.87) (width 0.2) (layer "F.Cu") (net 8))
 (segment (start 158.96 109.55) (end 158.96 108.94) (width 0.2) (layer "F.Cu") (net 8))
 (segment (start 151.34 116.634) (end 152.516 117.81) (width 0.2) (layer "B.Cu") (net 10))
 (segment (start 144.723115 128.24) (end 144.2 128.24) (width 0.2) (layer "B.Cu") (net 10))
 (segment (start 152.516 117.81) (end 152.516 120.447115) (width 0.2) (layer "B.Cu") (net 10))
 (segment (start 152.516 120.447115) (end 144.723115 128.24) (width 0.2) (layer "B.Cu") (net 10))
 (segment (start 151.34 109.55) (end 151.34 116.634) (width 0.2) (layer "B.Cu") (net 10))
 (segment (start 128.96 115.54) (end 127.985 114.565) (width 0.2) (layer "B.Cu") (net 17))
 (segment (start 132.12 81.07) (end 144.1 81.07) (width 0.2) (layer "B.Cu") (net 17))
 (segment (start 127.985 114.565) (end 127.985 85.205) (width 0.2) (layer "B.Cu") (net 17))
 (segment (start 127.985 85.205) (end 132.12 81.07) (width 0.2) (layer "B.Cu") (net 17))
 (segment (start 144.1 81.07) (end 144.19 80.98) (width 0.2) (layer "B.Cu") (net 17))
 (segment (start 141.67 126.62) (end 142.59 125.7) (width 0.2) (layer "B.Cu") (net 9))
 (segment (start 142.59 125.7) (end 144.2 125.7) (width 0.2) (layer "B.Cu") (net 9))
 (segment (start 155.056 110.726) (end 155.056 120.447115) (width 0.2) (layer "B.Cu") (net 9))
 (segment (start 141.67 127.84) (end 141.67 126.62) (width 0.2) (layer "B.Cu") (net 9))
 (segment (start 146.288115 129.215) (end 143.18 129.215) (width 0.2) (layer "B.Cu") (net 9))
 (segment (start 153.88 109.55) (end 155.056 110.726) (width 0.2) (layer "B.Cu") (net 9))
 (segment (start 141.67 127.84) (end 143.045 129.215) (width 0.2) (layer "B.Cu") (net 9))
 (segment (start 143.045 129.215) (end 143.18 129.215) (width 0.2) (layer "B.Cu") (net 9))
 (segment (start 155.056 120.447115) (end 146.288115 129.215) (width 0.2) (layer "B.Cu") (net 9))
 (segment (start 169.5 117.26) (end 169.5 117.38) (width 0.2) (layer "F.Cu") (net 2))
 (segment (start 169.09 116.85) (end 169.5 117.26) (width 0.2) (layer "F.Cu") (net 2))
 (segment (start 131.77 118.08) (end 133 116.85) (width 0.2) (layer "F.Cu") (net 2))
 (segment (start 133 116.85) (end 169.09 116.85) (width 0.2) (layer "F.Cu") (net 2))
 (segment (start 128.96 118.08) (end 131.77 118.08) (width 0.2) (layer "F.Cu") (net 2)))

